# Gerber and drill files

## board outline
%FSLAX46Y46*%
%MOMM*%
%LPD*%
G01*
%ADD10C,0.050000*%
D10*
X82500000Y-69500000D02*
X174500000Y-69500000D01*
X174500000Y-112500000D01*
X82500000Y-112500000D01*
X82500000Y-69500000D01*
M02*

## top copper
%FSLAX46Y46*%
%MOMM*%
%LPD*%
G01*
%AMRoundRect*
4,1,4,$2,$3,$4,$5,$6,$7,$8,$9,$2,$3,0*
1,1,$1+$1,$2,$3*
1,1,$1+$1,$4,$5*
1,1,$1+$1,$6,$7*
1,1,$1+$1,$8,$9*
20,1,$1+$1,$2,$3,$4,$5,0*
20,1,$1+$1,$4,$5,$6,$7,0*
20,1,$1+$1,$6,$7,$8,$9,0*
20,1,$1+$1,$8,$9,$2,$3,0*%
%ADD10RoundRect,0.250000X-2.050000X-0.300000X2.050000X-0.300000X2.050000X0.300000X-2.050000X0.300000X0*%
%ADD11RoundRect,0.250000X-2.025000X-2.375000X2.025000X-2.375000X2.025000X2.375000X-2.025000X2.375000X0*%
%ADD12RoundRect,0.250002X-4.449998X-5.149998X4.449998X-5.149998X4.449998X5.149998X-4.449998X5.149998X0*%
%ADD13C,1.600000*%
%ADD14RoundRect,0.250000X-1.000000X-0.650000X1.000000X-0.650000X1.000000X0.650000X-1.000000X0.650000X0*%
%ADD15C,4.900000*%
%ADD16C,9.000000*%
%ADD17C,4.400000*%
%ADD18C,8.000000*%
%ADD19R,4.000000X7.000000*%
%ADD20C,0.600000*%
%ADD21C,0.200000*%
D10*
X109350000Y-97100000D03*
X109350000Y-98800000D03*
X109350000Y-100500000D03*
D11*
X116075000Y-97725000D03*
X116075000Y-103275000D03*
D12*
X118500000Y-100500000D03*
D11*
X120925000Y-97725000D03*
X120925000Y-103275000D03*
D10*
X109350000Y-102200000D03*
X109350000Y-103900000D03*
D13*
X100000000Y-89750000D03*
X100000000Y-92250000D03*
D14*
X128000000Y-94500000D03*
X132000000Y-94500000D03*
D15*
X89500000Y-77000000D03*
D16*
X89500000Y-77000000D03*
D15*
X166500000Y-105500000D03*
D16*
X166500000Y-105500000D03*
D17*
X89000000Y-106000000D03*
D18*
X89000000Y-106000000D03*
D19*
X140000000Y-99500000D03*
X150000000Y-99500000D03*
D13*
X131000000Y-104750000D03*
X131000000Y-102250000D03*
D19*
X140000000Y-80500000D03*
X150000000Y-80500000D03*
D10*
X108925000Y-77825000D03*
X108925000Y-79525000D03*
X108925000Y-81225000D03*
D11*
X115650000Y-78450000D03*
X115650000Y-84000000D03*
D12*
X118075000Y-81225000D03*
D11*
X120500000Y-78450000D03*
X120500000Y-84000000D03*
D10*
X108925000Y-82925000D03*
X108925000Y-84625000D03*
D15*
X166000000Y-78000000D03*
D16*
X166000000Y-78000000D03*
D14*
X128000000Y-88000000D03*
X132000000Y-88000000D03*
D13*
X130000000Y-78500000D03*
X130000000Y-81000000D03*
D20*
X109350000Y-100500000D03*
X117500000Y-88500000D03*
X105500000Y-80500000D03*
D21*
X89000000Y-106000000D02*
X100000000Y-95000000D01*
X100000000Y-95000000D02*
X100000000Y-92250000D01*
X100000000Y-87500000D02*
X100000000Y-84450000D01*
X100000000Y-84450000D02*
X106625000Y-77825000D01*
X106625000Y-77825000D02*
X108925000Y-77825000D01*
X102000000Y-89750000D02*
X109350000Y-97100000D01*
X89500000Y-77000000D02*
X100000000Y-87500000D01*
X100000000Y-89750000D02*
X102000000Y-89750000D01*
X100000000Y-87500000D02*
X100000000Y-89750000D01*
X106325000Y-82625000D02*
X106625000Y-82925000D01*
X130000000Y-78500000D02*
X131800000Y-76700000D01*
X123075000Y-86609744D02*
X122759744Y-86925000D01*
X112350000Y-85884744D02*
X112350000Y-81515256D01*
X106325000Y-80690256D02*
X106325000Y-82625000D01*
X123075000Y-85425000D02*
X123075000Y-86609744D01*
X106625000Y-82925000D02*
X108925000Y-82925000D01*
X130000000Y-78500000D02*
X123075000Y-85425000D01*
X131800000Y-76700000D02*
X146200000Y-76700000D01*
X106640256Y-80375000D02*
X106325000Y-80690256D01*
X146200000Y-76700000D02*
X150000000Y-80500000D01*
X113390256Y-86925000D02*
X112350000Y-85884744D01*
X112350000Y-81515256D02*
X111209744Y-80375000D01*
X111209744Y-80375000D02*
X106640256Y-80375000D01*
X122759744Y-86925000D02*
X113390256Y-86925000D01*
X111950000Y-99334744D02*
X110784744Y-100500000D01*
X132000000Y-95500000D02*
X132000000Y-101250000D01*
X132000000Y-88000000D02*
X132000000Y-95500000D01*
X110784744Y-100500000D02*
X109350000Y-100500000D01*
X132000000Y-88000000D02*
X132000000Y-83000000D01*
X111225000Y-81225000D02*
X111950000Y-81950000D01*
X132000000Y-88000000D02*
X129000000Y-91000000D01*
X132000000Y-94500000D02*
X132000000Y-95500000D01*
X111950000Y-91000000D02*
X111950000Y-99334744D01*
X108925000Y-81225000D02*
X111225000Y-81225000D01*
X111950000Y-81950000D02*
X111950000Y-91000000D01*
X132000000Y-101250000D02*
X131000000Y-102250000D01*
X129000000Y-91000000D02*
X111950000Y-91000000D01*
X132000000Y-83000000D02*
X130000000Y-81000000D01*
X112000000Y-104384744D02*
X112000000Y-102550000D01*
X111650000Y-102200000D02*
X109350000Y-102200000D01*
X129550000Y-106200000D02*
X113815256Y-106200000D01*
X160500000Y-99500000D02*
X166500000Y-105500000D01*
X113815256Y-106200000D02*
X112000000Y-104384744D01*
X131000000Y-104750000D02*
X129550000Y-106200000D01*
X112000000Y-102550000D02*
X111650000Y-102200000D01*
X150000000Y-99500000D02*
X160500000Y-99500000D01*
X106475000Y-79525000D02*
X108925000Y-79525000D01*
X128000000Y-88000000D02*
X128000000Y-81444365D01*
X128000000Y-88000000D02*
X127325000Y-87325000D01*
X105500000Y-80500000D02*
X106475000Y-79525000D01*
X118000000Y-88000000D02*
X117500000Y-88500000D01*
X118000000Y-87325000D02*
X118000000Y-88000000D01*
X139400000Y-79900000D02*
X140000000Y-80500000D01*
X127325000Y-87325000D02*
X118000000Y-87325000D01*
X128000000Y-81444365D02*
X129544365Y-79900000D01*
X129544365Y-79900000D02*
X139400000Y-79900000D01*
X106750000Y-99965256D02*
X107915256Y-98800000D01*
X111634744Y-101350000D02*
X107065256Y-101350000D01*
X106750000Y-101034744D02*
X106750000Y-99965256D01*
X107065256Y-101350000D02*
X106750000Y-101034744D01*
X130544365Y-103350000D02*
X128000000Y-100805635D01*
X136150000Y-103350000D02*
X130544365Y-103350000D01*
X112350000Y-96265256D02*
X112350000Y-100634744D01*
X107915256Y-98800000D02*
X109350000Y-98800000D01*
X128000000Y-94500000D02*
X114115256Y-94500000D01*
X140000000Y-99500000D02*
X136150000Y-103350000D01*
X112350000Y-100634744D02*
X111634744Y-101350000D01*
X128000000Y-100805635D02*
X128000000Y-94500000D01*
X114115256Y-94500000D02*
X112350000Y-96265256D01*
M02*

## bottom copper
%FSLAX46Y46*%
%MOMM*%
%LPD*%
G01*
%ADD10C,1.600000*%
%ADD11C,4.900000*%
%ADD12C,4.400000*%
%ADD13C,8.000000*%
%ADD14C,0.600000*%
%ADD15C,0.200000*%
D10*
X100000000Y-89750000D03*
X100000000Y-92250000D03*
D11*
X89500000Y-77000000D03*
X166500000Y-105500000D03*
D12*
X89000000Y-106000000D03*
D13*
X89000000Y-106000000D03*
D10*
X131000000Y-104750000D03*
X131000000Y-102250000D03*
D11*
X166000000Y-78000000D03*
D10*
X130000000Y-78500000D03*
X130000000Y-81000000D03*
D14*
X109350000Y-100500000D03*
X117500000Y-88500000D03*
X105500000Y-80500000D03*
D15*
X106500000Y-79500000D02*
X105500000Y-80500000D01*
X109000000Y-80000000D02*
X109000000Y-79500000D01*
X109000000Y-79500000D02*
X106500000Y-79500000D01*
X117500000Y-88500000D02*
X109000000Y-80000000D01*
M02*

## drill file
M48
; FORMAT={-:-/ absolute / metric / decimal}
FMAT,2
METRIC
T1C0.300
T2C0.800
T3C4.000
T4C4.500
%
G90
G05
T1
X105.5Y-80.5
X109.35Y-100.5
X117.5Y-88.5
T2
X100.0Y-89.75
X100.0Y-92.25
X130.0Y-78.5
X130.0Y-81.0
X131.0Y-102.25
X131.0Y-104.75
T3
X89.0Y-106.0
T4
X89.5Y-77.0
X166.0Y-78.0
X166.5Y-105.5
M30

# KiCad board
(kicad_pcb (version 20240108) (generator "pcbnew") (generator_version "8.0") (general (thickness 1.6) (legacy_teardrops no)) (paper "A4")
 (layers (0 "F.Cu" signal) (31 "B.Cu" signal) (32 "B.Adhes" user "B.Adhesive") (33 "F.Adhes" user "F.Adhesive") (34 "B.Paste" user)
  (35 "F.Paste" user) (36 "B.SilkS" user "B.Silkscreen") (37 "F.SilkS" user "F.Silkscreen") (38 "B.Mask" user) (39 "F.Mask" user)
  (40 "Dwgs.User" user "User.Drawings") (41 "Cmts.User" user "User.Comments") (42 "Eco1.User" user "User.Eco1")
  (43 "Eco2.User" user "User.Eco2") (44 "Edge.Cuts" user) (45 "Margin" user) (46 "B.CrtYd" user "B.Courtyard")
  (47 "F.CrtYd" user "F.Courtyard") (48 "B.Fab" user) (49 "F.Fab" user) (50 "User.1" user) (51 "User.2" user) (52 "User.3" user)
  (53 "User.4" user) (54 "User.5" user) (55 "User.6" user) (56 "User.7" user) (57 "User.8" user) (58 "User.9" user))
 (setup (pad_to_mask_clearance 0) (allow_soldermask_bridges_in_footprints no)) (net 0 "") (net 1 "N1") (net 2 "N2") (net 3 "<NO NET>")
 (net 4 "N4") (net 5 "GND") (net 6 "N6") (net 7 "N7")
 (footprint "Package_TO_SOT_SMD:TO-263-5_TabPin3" (layer "F.Cu") (at 117 100.5)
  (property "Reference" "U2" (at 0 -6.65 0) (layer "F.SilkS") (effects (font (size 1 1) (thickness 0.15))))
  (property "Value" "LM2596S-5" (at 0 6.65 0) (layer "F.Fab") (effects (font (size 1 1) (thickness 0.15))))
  (pad "1" smd roundrect (at -7.65 -3.4) (size 4.6 1.1) (layers "F.Cu" "F.Paste" "F.Mask") (roundrect_rratio 0.227273) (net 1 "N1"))
  (pad "2" smd roundrect (at -7.65 -1.7) (size 4.6 1.1) (layers "F.Cu" "F.Paste" "F.Mask") (roundrect_rratio 0.227273) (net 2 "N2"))
  (pad "3" smd roundrect (at -7.65 0) (size 4.6 1.1) (layers "F.Cu" "F.Paste" "F.Mask") (roundrect_rratio 0.227273) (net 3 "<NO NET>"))
  (pad "3" smd roundrect (at -0.925 -2.775) (size 4.55 5.25) (layers "F.Cu" "F.Paste") (roundrect_rratio 0.054945) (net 3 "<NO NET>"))
  (pad "3" smd roundrect (at -0.925 2.775) (size 4.55 5.25) (layers "F.Cu" "F.Paste") (roundrect_rratio 0.054945) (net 3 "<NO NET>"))
  (pad "3" smd roundrect (at 1.5 0) (size 9.4 10.8) (layers "F.Cu" "F.Mask") (roundrect_rratio 0.026596) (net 3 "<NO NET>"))
  (pad "3" smd roundrect (at 3.925 -2.775) (size 4.55 5.25) (layers "F.Cu" "F.Paste") (roundrect_rratio 0.054945) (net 3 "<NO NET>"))
  (pad "3" smd roundrect (at 3.925 2.775) (size 4.55 5.25) (layers "F.Cu" "F.Paste") (roundrect_rratio 0.054945) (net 3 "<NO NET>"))
  (pad "4" smd roundrect (at -7.65 1.7) (size 4.6 1.1) (layers "F.Cu" "F.Paste" "F.Mask") (roundrect_rratio 0.227273) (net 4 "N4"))
  (pad "5" smd roundrect (at -7.65 3.4) (size 4.6 1.1) (layers "F.Cu" "F.Paste" "F.Mask") (roundrect_rratio 0.227273) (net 3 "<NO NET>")))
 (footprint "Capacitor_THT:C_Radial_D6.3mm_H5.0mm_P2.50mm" (layer "F.Cu") (at 100 89.75 -90)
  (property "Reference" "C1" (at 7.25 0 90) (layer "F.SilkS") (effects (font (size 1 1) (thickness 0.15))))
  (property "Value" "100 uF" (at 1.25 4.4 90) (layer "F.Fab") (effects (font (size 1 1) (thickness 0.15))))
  (pad "1" thru_hole circle (at 0 0 270) (size 1.6 1.6) (drill 0.8) (layers "*.Cu" "*.Mask") (remove_unused_layers no) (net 1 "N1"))
  (pad "2" thru_hole circle (at 2.5 0 270) (size 1.6 1.6) (drill 0.8) (layers "*.Cu" "*.Mask") (remove_unused_layers no) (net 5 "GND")))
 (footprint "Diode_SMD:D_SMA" (layer "F.Cu") (at 130 94.5)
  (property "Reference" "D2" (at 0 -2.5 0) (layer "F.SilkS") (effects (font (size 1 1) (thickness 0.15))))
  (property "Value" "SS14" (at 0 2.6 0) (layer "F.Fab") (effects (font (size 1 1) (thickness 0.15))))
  (pad "1" smd roundrect (at -2 0) (size 2.5 1.8) (layers "F.Cu" "F.Paste" "F.Mask") (roundrect_rratio 0.1388888889) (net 2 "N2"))
  (pad "2" smd roundrect (at 2 0) (size 2.5 1.8) (layers "F.Cu" "F.Paste" "F.Mask") (roundrect_rratio 0.1388888889) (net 3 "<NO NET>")))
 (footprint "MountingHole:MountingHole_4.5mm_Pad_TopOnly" (layer "F.Cu") (at 89.5 77)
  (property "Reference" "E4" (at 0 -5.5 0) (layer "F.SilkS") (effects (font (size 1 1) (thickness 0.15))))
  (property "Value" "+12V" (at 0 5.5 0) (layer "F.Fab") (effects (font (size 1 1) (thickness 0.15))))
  (pad "1" thru_hole circle (at 0 0) (size 4.9 4.9) (drill 4.5) (layers "*.Cu" "*.Mask") (remove_unused_layers no) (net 1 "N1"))
  (pad "1" connect circle (at 0 0) (size 9 9) (layers "F.Cu" "F.Mask") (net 1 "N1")))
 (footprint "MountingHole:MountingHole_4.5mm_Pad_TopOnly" (layer "F.Cu") (at 166.5 105.5)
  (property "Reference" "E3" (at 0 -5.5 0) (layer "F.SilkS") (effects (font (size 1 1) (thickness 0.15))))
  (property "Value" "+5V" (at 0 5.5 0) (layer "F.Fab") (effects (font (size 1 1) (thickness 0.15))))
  (pad "1" thru_hole circle (at 0 0) (size 4.9 4.9) (drill 4.5) (layers "*.Cu" "*.Mask") (remove_unused_layers no) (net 4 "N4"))
  (pad "1" connect circle (at 0 0) (size 9 9) (layers "F.Cu" "F.Mask") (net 4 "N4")))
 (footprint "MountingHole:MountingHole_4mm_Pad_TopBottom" (layer "F.Cu") (at 89 106)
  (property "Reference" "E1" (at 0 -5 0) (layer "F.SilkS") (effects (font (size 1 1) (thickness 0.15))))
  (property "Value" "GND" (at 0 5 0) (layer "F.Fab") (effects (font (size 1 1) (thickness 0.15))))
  (pad "1" thru_hole circle (at 0 0) (size 4.4 4.4) (drill 4) (layers "*.Cu" "*.Mask") (remove_unused_layers no) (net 5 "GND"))
  (pad "1" connect circle (at 0 0) (size 8 8) (layers "F.Cu" "F.Mask") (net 5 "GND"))
  (pad "1" connect circle (at 0 0) (size 8 8) (layers "B.Cu" "B.Mask") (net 5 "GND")))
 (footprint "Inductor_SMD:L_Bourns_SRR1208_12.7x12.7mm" (layer "F.Cu") (at 145 99.5)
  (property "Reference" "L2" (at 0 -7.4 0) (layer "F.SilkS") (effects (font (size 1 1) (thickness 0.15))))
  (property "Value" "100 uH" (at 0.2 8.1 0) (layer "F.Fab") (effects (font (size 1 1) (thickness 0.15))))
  (pad "1" smd rect (at -5 0) (size 4 7) (layers "F.Cu" "F.Paste" "F.Mask") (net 2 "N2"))
  (pad "2" smd rect (at 5 0) (size 4 7) (layers "F.Cu" "F.Paste" "F.Mask") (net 4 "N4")))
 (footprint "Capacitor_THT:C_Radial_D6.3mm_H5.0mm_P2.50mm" (layer "F.Cu") (at 131 104.75 90)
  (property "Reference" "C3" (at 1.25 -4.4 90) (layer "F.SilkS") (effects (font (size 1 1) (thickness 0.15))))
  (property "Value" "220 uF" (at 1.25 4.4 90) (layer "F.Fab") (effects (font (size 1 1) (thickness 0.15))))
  (pad "1" thru_hole circle (at 0 0 90) (size 1.6 1.6) (drill 0.8) (layers "*.Cu" "*.Mask") (remove_unused_layers no) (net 4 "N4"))
  (pad "2" thru_hole circle (at 2.5 0 90) (size 1.6 1.6) (drill 0.8) (layers "*.Cu" "*.Mask") (remove_unused_layers no) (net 3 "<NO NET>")))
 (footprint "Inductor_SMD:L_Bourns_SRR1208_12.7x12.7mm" (layer "F.Cu") (at 145 80.5)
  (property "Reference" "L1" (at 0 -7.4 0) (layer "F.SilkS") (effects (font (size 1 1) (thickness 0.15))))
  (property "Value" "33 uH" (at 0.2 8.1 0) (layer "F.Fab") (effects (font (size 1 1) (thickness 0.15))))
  (pad "1" smd rect (at -5 0) (size 4 7) (layers "F.Cu" "F.Paste" "F.Mask") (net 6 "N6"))
  (pad "2" smd rect (at 5 0) (size 4 7) (layers "F.Cu" "F.Paste" "F.Mask") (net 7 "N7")))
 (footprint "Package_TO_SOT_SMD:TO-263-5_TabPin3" (layer "F.Cu") (at 116.575 81.225)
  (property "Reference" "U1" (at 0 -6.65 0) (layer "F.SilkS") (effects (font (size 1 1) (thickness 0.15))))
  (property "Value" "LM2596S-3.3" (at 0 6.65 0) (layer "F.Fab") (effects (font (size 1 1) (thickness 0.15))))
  (pad "1" smd roundrect (at -7.65 -3.4) (size 4.6 1.1) (layers "F.Cu" "F.Paste" "F.Mask") (roundrect_rratio 0.227273) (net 1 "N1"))
  (pad "2" smd roundrect (at -7.65 -1.7) (size 4.6 1.1) (layers "F.Cu" "F.Paste" "F.Mask") (roundrect_rratio 0.227273) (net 6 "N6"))
  (pad "3" smd roundrect (at -7.65 0) (size 4.6 1.1) (layers "F.Cu" "F.Paste" "F.Mask") (roundrect_rratio 0.227273) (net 3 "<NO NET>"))
  (pad "3" smd roundrect (at -0.925 -2.775) (size 4.55 5.25) (layers "F.Cu" "F.Paste") (roundrect_rratio 0.054945) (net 3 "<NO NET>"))
  (pad "3" smd roundrect (at -0.925 2.775) (size 4.55 5.25) (layers "F.Cu" "F.Paste") (roundrect_rratio 0.054945) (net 3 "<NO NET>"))
  (pad "3" smd roundrect (at 1.5 0) (size 9.4 10.8) (layers "F.Cu" "F.Mask") (roundrect_rratio 0.026596) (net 3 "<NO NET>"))
  (pad "3" smd roundrect (at 3.925 -2.775) (size 4.55 5.25) (layers "F.Cu" "F.Paste") (roundrect_rratio 0.054945) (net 3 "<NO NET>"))
  (pad "3" smd roundrect (at 3.925 2.775) (size 4.55 5.25) (layers "F.Cu" "F.Paste") (roundrect_rratio 0.054945) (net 3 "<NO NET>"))
  (pad "4" smd roundrect (at -7.65 1.7) (size 4.6 1.1) (layers "F.Cu" "F.Paste" "F.Mask") (roundrect_rratio 0.227273) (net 7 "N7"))
  (pad "5" smd roundrect (at -7.65 3.4) (size 4.6 1.1) (layers "F.Cu" "F.Paste" "F.Mask") (roundrect_rratio 0.227273) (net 3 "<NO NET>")))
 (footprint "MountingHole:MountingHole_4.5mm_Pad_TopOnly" (layer "F.Cu") (at 166 78)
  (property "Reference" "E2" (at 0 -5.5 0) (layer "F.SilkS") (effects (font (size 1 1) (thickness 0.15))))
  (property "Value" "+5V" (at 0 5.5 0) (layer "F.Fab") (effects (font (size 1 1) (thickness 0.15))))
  (pad "1" thru_hole circle (at 0 0) (size 4.9 4.9) (drill 4.5) (layers "*.Cu" "*.Mask") (remove_unused_layers no) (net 7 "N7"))
  (pad "1" connect circle (at 0 0) (size 9 9) (layers "F.Cu" "F.Mask") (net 7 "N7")))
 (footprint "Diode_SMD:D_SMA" (layer "F.Cu") (at 130 88)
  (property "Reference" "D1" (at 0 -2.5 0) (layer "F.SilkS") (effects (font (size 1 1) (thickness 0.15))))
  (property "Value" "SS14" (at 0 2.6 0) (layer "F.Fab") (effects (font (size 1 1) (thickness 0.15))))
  (pad "1" smd roundrect (at -2 0) (size 2.5 1.8) (layers "F.Cu" "F.Paste" "F.Mask") (roundrect_rratio 0.1388888889) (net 6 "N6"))
  (pad "2" smd roundrect (at 2 0) (size 2.5 1.8) (layers "F.Cu" "F.Paste" "F.Mask") (roundrect_rratio 0.1388888889) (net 3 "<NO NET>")))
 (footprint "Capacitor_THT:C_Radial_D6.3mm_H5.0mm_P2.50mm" (layer "F.Cu") (at 130 78.5 -90)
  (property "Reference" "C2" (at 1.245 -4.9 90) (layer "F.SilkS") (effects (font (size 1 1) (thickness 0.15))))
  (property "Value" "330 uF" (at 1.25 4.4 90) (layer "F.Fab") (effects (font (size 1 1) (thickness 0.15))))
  (pad "1" thru_hole circle (at 0 0 270) (size 1.6 1.6) (drill 0.8) (layers "*.Cu" "*.Mask") (remove_unused_layers no) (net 7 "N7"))
  (pad "2" thru_hole circle (at 2.5 0 270) (size 1.6 1.6) (drill 0.8) (layers "*.Cu" "*.Mask") (remove_unused_layers no) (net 3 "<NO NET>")))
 (gr_rect (start 82.5 69.5) (end 174.5 112.5) (stroke (width 0.05) (type default)) (fill none) (layer "Edge.Cuts"))
 (segment (start 89 106) (end 100 95) (width 0.2) (layer "F.Cu") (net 5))
 (segment (start 100 95) (end 100 92.25) (width 0.2) (layer "F.Cu") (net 5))
 (segment (start 100 87.5) (end 100 84.45) (width 0.2) (layer "F.Cu") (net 1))
 (segment (start 100 84.45) (end 106.625 77.825) (width 0.2) (layer "F.Cu") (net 1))
 (segment (start 106.625 77.825) (end 108.925 77.825) (width 0.2) (layer "F.Cu") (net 1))
 (segment (start 102 89.75) (end 109.35 97.1) (width 0.2) (layer "F.Cu") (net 1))
 (segment (start 89.5 77) (end 100 87.5) (width 0.2) (layer "F.Cu") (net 1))
 (segment (start 100 89.75) (end 102 89.75) (width 0.2) (layer "F.Cu") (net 1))
 (segment (start 100 87.5) (end 100 89.75) (width 0.2) (layer "F.Cu") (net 1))
 (segment (start 106.325 82.625) (end 106.625 82.925) (width 0.2) (layer "F.Cu") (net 7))
 (segment (start 130 78.5) (end 131.8 76.7) (width 0.2) (layer "F.Cu") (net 7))
 (segment (start 123.075 86.609744) (end 122.759744 86.925) (width 0.2) (layer "F.Cu") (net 7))
 (segment (start 112.35 85.884744) (end 112.35 81.515256) (width 0.2) (layer "F.Cu") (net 7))
 (segment (start 106.325 80.690256) (end 106.325 82.625) (width 0.2) (layer "F.Cu") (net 7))
 (segment (start 123.075 85.425) (end 123.075 86.609744) (width 0.2) (layer "F.Cu") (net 7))
 (segment (start 106.625 82.925) (end 108.925 82.925) (width 0.2) (layer "F.Cu") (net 7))
 (segment (start 130 78.5) (end 123.075 85.425) (width 0.2) (layer "F.Cu") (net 7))
 (segment (start 131.8 76.7) (end 146.2 76.7) (width 0.2) (layer "F.Cu") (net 7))
 (segment (start 106.640256 80.375) (end 106.325 80.690256) (width 0.2) (layer "F.Cu") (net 7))
 (segment (start 146.2 76.7) (end 150 80.5) (width 0.2) (layer "F.Cu") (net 7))
 (segment (start 113.390256 86.925) (end 112.35 85.884744) (width 0.2) (layer "F.Cu") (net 7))
 (segment (start 112.35 81.515256) (end 111.209744 80.375) (width 0.2) (layer "F.Cu") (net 7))
 (segment (start 111.209744 80.375) (end 106.640256 80.375) (width 0.2) (layer "F.Cu") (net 7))
 (segment (start 122.759744 86.925) (end 113.390256 86.925) (width 0.2) (layer "F.Cu") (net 7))
 (segment (start 111.95 99.334744) (end 110.784744 100.5) (width 0.2) (layer "F.Cu") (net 3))
 (segment (start 132 95.5) (end 132 101.25) (width 0.2) (layer "F.Cu") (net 3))
 (segment (start 132 88) (end 132 95.5) (width 0.2) (layer "F.Cu") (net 3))
 (segment (start 110.784744 100.5) (end 109.35 100.5) (width 0.2) (layer "F.Cu") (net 3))
 (segment (start 132 88) (end 132 83) (width 0.2) (layer "F.Cu") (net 3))
 (segment (start 111.225 81.225) (end 111.95 81.95) (width 0.2) (layer "F.Cu") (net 3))
 (segment (start 132 88) (end 129 91) (width 0.2) (layer "F.Cu") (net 3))
 (segment (start 132 94.5) (end 132 95.5) (width 0.2) (layer "F.Cu") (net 3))
 (segment (start 111.95 91) (end 111.95 99.334744) (width 0.2) (layer "F.Cu") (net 3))
 (segment (start 108.925 81.225) (end 111.225 81.225) (width 0.2) (layer "F.Cu") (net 3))
 (segment (start 111.95 81.95) (end 111.95 91) (width 0.2) (layer "F.Cu") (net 3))
 (segment (start 132 101.25) (end 131 102.25) (width 0.2) (layer "F.Cu") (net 3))
 (segment (start 129 91) (end 111.95 91) (width 0.2) (layer "F.Cu") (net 3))
 (segment (start 132 83) (end 130 81) (width 0.2) (layer "F.Cu") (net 3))
 (via (at 109.35 100.5) (size 0.6) (drill 0.3) (layers "F.Cu" "B.Cu") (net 3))
 (segment (start 112 104.384744) (end 112 102.55) (width 0.2) (layer "F.Cu") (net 4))
 (segment (start 111.65 102.2) (end 109.35 102.2) (width 0.2) (layer "F.Cu") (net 4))
 (segment (start 129.55 106.2) (end 113.815256 106.2) (width 0.2) (layer "F.Cu") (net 4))
 (segment (start 160.5 99.5) (end 166.5 105.5) (width 0.2) (layer "F.Cu") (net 4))
 (segment (start 113.815256 106.2) (end 112 104.384744) (width 0.2) (layer "F.Cu") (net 4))
 (segment (start 131 104.75) (end 129.55 106.2) (width 0.2) (layer "F.Cu") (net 4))
 (segment (start 112 102.55) (end 111.65 102.2) (width 0.2) (layer "F.Cu") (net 4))
 (segment (start 150 99.5) (end 160.5 99.5) (width 0.2) (layer "F.Cu") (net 4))
 (segment (start 106.475 79.525) (end 108.925 79.525) (width 0.2) (layer "F.Cu") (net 6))
 (segment (start 128 88) (end 128 81.444365) (width 0.2) (layer "F.Cu") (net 6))
 (segment (start 128 88) (end 127.325 87.325) (width 0.2) (layer "F.Cu") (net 6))
 (segment (start 105.5 80.5) (end 106.475 79.525) (width 0.2) (layer "F.Cu") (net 6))
 (segment (start 118 88) (end 117.5 88.5) (width 0.2) (layer "F.Cu") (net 6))
 (segment (start 118 87.325) (end 118 88) (width 0.2) (layer "F.Cu") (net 6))
 (segment (start 139.4 79.9) (end 140 80.5) (width 0.2) (layer "F.Cu") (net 6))
 (segment (start 127.325 87.325) (end 118 87.325) (width 0.2) (layer "F.Cu") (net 6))
 (segment (start 128 81.444365) (end 129.544365 79.9) (width 0.2) (layer "F.Cu") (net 6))
 (segment (start 129.544365 79.9) (end 139.4 79.9) (width 0.2) (layer "F.Cu") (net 6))
 (via (at 117.5 88.5) (size 0.6) (drill 0.3) (layers "F.Cu" "B.Cu") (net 6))
 (via (at 105.5 80.5) (size 0.6) (drill 0.3) (layers "F.Cu" "B.Cu") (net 6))
 (segment (start 106.5 79.5) (end 105.5 80.5) (width 0.2) (layer "B.Cu") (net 6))
 (segment (start 109 80) (end 109 79.5) (width 0.2) (layer "B.Cu") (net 6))
 (segment (start 109 79.5) (end 106.5 79.5) (width 0.2) (layer "B.Cu") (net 6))
 (segment (start 117.5 88.5) (end 109 80) (width 0.2) (layer "B.Cu") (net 6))
 (segment (start 106.75 99.965256) (end 107.915256 98.8) (width 0.2) (layer "F.Cu") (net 2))
 (segment (start 111.634744 101.35) (end 107.065256 101.35) (width 0.2) (layer "F.Cu") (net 2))
 (segment (start 106.75 101.034744) (end 106.75 99.965256) (width 0.2) (layer "F.Cu") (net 2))
 (segment (start 107.065256 101.35) (end 106.75 101.034744) (width 0.2) (layer "F.Cu") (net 2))
 (segment (start 130.544365 103.35) (end 128 100.805635) (width 0.2) (layer "F.Cu") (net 2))
 (segment (start 136.15 103.35) (end 130.544365 103.35) (width 0.2) (layer "F.Cu") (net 2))
 (segment (start 112.35 96.265256) (end 112.35 100.634744) (width 0.2) (layer "F.Cu") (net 2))
 (segment (start 107.915256 98.8) (end 109.35 98.8) (width 0.2) (layer "F.Cu") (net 2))
 (segment (start 128 94.5) (end 114.115256 94.5) (width 0.2) (layer "F.Cu") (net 2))
 (segment (start 140 99.5) (end 136.15 103.35) (width 0.2) (layer "F.Cu") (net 2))
 (segment (start 112.35 100.634744) (end 111.634744 101.35) (width 0.2) (layer "F.Cu") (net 2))
 (segment (start 128 100.805635) (end 128 94.5) (width 0.2) (layer "F.Cu") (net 2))
 (segment (start 114.115256 94.5) (end 112.35 96.265256) (width 0.2) (layer "F.Cu") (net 2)))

